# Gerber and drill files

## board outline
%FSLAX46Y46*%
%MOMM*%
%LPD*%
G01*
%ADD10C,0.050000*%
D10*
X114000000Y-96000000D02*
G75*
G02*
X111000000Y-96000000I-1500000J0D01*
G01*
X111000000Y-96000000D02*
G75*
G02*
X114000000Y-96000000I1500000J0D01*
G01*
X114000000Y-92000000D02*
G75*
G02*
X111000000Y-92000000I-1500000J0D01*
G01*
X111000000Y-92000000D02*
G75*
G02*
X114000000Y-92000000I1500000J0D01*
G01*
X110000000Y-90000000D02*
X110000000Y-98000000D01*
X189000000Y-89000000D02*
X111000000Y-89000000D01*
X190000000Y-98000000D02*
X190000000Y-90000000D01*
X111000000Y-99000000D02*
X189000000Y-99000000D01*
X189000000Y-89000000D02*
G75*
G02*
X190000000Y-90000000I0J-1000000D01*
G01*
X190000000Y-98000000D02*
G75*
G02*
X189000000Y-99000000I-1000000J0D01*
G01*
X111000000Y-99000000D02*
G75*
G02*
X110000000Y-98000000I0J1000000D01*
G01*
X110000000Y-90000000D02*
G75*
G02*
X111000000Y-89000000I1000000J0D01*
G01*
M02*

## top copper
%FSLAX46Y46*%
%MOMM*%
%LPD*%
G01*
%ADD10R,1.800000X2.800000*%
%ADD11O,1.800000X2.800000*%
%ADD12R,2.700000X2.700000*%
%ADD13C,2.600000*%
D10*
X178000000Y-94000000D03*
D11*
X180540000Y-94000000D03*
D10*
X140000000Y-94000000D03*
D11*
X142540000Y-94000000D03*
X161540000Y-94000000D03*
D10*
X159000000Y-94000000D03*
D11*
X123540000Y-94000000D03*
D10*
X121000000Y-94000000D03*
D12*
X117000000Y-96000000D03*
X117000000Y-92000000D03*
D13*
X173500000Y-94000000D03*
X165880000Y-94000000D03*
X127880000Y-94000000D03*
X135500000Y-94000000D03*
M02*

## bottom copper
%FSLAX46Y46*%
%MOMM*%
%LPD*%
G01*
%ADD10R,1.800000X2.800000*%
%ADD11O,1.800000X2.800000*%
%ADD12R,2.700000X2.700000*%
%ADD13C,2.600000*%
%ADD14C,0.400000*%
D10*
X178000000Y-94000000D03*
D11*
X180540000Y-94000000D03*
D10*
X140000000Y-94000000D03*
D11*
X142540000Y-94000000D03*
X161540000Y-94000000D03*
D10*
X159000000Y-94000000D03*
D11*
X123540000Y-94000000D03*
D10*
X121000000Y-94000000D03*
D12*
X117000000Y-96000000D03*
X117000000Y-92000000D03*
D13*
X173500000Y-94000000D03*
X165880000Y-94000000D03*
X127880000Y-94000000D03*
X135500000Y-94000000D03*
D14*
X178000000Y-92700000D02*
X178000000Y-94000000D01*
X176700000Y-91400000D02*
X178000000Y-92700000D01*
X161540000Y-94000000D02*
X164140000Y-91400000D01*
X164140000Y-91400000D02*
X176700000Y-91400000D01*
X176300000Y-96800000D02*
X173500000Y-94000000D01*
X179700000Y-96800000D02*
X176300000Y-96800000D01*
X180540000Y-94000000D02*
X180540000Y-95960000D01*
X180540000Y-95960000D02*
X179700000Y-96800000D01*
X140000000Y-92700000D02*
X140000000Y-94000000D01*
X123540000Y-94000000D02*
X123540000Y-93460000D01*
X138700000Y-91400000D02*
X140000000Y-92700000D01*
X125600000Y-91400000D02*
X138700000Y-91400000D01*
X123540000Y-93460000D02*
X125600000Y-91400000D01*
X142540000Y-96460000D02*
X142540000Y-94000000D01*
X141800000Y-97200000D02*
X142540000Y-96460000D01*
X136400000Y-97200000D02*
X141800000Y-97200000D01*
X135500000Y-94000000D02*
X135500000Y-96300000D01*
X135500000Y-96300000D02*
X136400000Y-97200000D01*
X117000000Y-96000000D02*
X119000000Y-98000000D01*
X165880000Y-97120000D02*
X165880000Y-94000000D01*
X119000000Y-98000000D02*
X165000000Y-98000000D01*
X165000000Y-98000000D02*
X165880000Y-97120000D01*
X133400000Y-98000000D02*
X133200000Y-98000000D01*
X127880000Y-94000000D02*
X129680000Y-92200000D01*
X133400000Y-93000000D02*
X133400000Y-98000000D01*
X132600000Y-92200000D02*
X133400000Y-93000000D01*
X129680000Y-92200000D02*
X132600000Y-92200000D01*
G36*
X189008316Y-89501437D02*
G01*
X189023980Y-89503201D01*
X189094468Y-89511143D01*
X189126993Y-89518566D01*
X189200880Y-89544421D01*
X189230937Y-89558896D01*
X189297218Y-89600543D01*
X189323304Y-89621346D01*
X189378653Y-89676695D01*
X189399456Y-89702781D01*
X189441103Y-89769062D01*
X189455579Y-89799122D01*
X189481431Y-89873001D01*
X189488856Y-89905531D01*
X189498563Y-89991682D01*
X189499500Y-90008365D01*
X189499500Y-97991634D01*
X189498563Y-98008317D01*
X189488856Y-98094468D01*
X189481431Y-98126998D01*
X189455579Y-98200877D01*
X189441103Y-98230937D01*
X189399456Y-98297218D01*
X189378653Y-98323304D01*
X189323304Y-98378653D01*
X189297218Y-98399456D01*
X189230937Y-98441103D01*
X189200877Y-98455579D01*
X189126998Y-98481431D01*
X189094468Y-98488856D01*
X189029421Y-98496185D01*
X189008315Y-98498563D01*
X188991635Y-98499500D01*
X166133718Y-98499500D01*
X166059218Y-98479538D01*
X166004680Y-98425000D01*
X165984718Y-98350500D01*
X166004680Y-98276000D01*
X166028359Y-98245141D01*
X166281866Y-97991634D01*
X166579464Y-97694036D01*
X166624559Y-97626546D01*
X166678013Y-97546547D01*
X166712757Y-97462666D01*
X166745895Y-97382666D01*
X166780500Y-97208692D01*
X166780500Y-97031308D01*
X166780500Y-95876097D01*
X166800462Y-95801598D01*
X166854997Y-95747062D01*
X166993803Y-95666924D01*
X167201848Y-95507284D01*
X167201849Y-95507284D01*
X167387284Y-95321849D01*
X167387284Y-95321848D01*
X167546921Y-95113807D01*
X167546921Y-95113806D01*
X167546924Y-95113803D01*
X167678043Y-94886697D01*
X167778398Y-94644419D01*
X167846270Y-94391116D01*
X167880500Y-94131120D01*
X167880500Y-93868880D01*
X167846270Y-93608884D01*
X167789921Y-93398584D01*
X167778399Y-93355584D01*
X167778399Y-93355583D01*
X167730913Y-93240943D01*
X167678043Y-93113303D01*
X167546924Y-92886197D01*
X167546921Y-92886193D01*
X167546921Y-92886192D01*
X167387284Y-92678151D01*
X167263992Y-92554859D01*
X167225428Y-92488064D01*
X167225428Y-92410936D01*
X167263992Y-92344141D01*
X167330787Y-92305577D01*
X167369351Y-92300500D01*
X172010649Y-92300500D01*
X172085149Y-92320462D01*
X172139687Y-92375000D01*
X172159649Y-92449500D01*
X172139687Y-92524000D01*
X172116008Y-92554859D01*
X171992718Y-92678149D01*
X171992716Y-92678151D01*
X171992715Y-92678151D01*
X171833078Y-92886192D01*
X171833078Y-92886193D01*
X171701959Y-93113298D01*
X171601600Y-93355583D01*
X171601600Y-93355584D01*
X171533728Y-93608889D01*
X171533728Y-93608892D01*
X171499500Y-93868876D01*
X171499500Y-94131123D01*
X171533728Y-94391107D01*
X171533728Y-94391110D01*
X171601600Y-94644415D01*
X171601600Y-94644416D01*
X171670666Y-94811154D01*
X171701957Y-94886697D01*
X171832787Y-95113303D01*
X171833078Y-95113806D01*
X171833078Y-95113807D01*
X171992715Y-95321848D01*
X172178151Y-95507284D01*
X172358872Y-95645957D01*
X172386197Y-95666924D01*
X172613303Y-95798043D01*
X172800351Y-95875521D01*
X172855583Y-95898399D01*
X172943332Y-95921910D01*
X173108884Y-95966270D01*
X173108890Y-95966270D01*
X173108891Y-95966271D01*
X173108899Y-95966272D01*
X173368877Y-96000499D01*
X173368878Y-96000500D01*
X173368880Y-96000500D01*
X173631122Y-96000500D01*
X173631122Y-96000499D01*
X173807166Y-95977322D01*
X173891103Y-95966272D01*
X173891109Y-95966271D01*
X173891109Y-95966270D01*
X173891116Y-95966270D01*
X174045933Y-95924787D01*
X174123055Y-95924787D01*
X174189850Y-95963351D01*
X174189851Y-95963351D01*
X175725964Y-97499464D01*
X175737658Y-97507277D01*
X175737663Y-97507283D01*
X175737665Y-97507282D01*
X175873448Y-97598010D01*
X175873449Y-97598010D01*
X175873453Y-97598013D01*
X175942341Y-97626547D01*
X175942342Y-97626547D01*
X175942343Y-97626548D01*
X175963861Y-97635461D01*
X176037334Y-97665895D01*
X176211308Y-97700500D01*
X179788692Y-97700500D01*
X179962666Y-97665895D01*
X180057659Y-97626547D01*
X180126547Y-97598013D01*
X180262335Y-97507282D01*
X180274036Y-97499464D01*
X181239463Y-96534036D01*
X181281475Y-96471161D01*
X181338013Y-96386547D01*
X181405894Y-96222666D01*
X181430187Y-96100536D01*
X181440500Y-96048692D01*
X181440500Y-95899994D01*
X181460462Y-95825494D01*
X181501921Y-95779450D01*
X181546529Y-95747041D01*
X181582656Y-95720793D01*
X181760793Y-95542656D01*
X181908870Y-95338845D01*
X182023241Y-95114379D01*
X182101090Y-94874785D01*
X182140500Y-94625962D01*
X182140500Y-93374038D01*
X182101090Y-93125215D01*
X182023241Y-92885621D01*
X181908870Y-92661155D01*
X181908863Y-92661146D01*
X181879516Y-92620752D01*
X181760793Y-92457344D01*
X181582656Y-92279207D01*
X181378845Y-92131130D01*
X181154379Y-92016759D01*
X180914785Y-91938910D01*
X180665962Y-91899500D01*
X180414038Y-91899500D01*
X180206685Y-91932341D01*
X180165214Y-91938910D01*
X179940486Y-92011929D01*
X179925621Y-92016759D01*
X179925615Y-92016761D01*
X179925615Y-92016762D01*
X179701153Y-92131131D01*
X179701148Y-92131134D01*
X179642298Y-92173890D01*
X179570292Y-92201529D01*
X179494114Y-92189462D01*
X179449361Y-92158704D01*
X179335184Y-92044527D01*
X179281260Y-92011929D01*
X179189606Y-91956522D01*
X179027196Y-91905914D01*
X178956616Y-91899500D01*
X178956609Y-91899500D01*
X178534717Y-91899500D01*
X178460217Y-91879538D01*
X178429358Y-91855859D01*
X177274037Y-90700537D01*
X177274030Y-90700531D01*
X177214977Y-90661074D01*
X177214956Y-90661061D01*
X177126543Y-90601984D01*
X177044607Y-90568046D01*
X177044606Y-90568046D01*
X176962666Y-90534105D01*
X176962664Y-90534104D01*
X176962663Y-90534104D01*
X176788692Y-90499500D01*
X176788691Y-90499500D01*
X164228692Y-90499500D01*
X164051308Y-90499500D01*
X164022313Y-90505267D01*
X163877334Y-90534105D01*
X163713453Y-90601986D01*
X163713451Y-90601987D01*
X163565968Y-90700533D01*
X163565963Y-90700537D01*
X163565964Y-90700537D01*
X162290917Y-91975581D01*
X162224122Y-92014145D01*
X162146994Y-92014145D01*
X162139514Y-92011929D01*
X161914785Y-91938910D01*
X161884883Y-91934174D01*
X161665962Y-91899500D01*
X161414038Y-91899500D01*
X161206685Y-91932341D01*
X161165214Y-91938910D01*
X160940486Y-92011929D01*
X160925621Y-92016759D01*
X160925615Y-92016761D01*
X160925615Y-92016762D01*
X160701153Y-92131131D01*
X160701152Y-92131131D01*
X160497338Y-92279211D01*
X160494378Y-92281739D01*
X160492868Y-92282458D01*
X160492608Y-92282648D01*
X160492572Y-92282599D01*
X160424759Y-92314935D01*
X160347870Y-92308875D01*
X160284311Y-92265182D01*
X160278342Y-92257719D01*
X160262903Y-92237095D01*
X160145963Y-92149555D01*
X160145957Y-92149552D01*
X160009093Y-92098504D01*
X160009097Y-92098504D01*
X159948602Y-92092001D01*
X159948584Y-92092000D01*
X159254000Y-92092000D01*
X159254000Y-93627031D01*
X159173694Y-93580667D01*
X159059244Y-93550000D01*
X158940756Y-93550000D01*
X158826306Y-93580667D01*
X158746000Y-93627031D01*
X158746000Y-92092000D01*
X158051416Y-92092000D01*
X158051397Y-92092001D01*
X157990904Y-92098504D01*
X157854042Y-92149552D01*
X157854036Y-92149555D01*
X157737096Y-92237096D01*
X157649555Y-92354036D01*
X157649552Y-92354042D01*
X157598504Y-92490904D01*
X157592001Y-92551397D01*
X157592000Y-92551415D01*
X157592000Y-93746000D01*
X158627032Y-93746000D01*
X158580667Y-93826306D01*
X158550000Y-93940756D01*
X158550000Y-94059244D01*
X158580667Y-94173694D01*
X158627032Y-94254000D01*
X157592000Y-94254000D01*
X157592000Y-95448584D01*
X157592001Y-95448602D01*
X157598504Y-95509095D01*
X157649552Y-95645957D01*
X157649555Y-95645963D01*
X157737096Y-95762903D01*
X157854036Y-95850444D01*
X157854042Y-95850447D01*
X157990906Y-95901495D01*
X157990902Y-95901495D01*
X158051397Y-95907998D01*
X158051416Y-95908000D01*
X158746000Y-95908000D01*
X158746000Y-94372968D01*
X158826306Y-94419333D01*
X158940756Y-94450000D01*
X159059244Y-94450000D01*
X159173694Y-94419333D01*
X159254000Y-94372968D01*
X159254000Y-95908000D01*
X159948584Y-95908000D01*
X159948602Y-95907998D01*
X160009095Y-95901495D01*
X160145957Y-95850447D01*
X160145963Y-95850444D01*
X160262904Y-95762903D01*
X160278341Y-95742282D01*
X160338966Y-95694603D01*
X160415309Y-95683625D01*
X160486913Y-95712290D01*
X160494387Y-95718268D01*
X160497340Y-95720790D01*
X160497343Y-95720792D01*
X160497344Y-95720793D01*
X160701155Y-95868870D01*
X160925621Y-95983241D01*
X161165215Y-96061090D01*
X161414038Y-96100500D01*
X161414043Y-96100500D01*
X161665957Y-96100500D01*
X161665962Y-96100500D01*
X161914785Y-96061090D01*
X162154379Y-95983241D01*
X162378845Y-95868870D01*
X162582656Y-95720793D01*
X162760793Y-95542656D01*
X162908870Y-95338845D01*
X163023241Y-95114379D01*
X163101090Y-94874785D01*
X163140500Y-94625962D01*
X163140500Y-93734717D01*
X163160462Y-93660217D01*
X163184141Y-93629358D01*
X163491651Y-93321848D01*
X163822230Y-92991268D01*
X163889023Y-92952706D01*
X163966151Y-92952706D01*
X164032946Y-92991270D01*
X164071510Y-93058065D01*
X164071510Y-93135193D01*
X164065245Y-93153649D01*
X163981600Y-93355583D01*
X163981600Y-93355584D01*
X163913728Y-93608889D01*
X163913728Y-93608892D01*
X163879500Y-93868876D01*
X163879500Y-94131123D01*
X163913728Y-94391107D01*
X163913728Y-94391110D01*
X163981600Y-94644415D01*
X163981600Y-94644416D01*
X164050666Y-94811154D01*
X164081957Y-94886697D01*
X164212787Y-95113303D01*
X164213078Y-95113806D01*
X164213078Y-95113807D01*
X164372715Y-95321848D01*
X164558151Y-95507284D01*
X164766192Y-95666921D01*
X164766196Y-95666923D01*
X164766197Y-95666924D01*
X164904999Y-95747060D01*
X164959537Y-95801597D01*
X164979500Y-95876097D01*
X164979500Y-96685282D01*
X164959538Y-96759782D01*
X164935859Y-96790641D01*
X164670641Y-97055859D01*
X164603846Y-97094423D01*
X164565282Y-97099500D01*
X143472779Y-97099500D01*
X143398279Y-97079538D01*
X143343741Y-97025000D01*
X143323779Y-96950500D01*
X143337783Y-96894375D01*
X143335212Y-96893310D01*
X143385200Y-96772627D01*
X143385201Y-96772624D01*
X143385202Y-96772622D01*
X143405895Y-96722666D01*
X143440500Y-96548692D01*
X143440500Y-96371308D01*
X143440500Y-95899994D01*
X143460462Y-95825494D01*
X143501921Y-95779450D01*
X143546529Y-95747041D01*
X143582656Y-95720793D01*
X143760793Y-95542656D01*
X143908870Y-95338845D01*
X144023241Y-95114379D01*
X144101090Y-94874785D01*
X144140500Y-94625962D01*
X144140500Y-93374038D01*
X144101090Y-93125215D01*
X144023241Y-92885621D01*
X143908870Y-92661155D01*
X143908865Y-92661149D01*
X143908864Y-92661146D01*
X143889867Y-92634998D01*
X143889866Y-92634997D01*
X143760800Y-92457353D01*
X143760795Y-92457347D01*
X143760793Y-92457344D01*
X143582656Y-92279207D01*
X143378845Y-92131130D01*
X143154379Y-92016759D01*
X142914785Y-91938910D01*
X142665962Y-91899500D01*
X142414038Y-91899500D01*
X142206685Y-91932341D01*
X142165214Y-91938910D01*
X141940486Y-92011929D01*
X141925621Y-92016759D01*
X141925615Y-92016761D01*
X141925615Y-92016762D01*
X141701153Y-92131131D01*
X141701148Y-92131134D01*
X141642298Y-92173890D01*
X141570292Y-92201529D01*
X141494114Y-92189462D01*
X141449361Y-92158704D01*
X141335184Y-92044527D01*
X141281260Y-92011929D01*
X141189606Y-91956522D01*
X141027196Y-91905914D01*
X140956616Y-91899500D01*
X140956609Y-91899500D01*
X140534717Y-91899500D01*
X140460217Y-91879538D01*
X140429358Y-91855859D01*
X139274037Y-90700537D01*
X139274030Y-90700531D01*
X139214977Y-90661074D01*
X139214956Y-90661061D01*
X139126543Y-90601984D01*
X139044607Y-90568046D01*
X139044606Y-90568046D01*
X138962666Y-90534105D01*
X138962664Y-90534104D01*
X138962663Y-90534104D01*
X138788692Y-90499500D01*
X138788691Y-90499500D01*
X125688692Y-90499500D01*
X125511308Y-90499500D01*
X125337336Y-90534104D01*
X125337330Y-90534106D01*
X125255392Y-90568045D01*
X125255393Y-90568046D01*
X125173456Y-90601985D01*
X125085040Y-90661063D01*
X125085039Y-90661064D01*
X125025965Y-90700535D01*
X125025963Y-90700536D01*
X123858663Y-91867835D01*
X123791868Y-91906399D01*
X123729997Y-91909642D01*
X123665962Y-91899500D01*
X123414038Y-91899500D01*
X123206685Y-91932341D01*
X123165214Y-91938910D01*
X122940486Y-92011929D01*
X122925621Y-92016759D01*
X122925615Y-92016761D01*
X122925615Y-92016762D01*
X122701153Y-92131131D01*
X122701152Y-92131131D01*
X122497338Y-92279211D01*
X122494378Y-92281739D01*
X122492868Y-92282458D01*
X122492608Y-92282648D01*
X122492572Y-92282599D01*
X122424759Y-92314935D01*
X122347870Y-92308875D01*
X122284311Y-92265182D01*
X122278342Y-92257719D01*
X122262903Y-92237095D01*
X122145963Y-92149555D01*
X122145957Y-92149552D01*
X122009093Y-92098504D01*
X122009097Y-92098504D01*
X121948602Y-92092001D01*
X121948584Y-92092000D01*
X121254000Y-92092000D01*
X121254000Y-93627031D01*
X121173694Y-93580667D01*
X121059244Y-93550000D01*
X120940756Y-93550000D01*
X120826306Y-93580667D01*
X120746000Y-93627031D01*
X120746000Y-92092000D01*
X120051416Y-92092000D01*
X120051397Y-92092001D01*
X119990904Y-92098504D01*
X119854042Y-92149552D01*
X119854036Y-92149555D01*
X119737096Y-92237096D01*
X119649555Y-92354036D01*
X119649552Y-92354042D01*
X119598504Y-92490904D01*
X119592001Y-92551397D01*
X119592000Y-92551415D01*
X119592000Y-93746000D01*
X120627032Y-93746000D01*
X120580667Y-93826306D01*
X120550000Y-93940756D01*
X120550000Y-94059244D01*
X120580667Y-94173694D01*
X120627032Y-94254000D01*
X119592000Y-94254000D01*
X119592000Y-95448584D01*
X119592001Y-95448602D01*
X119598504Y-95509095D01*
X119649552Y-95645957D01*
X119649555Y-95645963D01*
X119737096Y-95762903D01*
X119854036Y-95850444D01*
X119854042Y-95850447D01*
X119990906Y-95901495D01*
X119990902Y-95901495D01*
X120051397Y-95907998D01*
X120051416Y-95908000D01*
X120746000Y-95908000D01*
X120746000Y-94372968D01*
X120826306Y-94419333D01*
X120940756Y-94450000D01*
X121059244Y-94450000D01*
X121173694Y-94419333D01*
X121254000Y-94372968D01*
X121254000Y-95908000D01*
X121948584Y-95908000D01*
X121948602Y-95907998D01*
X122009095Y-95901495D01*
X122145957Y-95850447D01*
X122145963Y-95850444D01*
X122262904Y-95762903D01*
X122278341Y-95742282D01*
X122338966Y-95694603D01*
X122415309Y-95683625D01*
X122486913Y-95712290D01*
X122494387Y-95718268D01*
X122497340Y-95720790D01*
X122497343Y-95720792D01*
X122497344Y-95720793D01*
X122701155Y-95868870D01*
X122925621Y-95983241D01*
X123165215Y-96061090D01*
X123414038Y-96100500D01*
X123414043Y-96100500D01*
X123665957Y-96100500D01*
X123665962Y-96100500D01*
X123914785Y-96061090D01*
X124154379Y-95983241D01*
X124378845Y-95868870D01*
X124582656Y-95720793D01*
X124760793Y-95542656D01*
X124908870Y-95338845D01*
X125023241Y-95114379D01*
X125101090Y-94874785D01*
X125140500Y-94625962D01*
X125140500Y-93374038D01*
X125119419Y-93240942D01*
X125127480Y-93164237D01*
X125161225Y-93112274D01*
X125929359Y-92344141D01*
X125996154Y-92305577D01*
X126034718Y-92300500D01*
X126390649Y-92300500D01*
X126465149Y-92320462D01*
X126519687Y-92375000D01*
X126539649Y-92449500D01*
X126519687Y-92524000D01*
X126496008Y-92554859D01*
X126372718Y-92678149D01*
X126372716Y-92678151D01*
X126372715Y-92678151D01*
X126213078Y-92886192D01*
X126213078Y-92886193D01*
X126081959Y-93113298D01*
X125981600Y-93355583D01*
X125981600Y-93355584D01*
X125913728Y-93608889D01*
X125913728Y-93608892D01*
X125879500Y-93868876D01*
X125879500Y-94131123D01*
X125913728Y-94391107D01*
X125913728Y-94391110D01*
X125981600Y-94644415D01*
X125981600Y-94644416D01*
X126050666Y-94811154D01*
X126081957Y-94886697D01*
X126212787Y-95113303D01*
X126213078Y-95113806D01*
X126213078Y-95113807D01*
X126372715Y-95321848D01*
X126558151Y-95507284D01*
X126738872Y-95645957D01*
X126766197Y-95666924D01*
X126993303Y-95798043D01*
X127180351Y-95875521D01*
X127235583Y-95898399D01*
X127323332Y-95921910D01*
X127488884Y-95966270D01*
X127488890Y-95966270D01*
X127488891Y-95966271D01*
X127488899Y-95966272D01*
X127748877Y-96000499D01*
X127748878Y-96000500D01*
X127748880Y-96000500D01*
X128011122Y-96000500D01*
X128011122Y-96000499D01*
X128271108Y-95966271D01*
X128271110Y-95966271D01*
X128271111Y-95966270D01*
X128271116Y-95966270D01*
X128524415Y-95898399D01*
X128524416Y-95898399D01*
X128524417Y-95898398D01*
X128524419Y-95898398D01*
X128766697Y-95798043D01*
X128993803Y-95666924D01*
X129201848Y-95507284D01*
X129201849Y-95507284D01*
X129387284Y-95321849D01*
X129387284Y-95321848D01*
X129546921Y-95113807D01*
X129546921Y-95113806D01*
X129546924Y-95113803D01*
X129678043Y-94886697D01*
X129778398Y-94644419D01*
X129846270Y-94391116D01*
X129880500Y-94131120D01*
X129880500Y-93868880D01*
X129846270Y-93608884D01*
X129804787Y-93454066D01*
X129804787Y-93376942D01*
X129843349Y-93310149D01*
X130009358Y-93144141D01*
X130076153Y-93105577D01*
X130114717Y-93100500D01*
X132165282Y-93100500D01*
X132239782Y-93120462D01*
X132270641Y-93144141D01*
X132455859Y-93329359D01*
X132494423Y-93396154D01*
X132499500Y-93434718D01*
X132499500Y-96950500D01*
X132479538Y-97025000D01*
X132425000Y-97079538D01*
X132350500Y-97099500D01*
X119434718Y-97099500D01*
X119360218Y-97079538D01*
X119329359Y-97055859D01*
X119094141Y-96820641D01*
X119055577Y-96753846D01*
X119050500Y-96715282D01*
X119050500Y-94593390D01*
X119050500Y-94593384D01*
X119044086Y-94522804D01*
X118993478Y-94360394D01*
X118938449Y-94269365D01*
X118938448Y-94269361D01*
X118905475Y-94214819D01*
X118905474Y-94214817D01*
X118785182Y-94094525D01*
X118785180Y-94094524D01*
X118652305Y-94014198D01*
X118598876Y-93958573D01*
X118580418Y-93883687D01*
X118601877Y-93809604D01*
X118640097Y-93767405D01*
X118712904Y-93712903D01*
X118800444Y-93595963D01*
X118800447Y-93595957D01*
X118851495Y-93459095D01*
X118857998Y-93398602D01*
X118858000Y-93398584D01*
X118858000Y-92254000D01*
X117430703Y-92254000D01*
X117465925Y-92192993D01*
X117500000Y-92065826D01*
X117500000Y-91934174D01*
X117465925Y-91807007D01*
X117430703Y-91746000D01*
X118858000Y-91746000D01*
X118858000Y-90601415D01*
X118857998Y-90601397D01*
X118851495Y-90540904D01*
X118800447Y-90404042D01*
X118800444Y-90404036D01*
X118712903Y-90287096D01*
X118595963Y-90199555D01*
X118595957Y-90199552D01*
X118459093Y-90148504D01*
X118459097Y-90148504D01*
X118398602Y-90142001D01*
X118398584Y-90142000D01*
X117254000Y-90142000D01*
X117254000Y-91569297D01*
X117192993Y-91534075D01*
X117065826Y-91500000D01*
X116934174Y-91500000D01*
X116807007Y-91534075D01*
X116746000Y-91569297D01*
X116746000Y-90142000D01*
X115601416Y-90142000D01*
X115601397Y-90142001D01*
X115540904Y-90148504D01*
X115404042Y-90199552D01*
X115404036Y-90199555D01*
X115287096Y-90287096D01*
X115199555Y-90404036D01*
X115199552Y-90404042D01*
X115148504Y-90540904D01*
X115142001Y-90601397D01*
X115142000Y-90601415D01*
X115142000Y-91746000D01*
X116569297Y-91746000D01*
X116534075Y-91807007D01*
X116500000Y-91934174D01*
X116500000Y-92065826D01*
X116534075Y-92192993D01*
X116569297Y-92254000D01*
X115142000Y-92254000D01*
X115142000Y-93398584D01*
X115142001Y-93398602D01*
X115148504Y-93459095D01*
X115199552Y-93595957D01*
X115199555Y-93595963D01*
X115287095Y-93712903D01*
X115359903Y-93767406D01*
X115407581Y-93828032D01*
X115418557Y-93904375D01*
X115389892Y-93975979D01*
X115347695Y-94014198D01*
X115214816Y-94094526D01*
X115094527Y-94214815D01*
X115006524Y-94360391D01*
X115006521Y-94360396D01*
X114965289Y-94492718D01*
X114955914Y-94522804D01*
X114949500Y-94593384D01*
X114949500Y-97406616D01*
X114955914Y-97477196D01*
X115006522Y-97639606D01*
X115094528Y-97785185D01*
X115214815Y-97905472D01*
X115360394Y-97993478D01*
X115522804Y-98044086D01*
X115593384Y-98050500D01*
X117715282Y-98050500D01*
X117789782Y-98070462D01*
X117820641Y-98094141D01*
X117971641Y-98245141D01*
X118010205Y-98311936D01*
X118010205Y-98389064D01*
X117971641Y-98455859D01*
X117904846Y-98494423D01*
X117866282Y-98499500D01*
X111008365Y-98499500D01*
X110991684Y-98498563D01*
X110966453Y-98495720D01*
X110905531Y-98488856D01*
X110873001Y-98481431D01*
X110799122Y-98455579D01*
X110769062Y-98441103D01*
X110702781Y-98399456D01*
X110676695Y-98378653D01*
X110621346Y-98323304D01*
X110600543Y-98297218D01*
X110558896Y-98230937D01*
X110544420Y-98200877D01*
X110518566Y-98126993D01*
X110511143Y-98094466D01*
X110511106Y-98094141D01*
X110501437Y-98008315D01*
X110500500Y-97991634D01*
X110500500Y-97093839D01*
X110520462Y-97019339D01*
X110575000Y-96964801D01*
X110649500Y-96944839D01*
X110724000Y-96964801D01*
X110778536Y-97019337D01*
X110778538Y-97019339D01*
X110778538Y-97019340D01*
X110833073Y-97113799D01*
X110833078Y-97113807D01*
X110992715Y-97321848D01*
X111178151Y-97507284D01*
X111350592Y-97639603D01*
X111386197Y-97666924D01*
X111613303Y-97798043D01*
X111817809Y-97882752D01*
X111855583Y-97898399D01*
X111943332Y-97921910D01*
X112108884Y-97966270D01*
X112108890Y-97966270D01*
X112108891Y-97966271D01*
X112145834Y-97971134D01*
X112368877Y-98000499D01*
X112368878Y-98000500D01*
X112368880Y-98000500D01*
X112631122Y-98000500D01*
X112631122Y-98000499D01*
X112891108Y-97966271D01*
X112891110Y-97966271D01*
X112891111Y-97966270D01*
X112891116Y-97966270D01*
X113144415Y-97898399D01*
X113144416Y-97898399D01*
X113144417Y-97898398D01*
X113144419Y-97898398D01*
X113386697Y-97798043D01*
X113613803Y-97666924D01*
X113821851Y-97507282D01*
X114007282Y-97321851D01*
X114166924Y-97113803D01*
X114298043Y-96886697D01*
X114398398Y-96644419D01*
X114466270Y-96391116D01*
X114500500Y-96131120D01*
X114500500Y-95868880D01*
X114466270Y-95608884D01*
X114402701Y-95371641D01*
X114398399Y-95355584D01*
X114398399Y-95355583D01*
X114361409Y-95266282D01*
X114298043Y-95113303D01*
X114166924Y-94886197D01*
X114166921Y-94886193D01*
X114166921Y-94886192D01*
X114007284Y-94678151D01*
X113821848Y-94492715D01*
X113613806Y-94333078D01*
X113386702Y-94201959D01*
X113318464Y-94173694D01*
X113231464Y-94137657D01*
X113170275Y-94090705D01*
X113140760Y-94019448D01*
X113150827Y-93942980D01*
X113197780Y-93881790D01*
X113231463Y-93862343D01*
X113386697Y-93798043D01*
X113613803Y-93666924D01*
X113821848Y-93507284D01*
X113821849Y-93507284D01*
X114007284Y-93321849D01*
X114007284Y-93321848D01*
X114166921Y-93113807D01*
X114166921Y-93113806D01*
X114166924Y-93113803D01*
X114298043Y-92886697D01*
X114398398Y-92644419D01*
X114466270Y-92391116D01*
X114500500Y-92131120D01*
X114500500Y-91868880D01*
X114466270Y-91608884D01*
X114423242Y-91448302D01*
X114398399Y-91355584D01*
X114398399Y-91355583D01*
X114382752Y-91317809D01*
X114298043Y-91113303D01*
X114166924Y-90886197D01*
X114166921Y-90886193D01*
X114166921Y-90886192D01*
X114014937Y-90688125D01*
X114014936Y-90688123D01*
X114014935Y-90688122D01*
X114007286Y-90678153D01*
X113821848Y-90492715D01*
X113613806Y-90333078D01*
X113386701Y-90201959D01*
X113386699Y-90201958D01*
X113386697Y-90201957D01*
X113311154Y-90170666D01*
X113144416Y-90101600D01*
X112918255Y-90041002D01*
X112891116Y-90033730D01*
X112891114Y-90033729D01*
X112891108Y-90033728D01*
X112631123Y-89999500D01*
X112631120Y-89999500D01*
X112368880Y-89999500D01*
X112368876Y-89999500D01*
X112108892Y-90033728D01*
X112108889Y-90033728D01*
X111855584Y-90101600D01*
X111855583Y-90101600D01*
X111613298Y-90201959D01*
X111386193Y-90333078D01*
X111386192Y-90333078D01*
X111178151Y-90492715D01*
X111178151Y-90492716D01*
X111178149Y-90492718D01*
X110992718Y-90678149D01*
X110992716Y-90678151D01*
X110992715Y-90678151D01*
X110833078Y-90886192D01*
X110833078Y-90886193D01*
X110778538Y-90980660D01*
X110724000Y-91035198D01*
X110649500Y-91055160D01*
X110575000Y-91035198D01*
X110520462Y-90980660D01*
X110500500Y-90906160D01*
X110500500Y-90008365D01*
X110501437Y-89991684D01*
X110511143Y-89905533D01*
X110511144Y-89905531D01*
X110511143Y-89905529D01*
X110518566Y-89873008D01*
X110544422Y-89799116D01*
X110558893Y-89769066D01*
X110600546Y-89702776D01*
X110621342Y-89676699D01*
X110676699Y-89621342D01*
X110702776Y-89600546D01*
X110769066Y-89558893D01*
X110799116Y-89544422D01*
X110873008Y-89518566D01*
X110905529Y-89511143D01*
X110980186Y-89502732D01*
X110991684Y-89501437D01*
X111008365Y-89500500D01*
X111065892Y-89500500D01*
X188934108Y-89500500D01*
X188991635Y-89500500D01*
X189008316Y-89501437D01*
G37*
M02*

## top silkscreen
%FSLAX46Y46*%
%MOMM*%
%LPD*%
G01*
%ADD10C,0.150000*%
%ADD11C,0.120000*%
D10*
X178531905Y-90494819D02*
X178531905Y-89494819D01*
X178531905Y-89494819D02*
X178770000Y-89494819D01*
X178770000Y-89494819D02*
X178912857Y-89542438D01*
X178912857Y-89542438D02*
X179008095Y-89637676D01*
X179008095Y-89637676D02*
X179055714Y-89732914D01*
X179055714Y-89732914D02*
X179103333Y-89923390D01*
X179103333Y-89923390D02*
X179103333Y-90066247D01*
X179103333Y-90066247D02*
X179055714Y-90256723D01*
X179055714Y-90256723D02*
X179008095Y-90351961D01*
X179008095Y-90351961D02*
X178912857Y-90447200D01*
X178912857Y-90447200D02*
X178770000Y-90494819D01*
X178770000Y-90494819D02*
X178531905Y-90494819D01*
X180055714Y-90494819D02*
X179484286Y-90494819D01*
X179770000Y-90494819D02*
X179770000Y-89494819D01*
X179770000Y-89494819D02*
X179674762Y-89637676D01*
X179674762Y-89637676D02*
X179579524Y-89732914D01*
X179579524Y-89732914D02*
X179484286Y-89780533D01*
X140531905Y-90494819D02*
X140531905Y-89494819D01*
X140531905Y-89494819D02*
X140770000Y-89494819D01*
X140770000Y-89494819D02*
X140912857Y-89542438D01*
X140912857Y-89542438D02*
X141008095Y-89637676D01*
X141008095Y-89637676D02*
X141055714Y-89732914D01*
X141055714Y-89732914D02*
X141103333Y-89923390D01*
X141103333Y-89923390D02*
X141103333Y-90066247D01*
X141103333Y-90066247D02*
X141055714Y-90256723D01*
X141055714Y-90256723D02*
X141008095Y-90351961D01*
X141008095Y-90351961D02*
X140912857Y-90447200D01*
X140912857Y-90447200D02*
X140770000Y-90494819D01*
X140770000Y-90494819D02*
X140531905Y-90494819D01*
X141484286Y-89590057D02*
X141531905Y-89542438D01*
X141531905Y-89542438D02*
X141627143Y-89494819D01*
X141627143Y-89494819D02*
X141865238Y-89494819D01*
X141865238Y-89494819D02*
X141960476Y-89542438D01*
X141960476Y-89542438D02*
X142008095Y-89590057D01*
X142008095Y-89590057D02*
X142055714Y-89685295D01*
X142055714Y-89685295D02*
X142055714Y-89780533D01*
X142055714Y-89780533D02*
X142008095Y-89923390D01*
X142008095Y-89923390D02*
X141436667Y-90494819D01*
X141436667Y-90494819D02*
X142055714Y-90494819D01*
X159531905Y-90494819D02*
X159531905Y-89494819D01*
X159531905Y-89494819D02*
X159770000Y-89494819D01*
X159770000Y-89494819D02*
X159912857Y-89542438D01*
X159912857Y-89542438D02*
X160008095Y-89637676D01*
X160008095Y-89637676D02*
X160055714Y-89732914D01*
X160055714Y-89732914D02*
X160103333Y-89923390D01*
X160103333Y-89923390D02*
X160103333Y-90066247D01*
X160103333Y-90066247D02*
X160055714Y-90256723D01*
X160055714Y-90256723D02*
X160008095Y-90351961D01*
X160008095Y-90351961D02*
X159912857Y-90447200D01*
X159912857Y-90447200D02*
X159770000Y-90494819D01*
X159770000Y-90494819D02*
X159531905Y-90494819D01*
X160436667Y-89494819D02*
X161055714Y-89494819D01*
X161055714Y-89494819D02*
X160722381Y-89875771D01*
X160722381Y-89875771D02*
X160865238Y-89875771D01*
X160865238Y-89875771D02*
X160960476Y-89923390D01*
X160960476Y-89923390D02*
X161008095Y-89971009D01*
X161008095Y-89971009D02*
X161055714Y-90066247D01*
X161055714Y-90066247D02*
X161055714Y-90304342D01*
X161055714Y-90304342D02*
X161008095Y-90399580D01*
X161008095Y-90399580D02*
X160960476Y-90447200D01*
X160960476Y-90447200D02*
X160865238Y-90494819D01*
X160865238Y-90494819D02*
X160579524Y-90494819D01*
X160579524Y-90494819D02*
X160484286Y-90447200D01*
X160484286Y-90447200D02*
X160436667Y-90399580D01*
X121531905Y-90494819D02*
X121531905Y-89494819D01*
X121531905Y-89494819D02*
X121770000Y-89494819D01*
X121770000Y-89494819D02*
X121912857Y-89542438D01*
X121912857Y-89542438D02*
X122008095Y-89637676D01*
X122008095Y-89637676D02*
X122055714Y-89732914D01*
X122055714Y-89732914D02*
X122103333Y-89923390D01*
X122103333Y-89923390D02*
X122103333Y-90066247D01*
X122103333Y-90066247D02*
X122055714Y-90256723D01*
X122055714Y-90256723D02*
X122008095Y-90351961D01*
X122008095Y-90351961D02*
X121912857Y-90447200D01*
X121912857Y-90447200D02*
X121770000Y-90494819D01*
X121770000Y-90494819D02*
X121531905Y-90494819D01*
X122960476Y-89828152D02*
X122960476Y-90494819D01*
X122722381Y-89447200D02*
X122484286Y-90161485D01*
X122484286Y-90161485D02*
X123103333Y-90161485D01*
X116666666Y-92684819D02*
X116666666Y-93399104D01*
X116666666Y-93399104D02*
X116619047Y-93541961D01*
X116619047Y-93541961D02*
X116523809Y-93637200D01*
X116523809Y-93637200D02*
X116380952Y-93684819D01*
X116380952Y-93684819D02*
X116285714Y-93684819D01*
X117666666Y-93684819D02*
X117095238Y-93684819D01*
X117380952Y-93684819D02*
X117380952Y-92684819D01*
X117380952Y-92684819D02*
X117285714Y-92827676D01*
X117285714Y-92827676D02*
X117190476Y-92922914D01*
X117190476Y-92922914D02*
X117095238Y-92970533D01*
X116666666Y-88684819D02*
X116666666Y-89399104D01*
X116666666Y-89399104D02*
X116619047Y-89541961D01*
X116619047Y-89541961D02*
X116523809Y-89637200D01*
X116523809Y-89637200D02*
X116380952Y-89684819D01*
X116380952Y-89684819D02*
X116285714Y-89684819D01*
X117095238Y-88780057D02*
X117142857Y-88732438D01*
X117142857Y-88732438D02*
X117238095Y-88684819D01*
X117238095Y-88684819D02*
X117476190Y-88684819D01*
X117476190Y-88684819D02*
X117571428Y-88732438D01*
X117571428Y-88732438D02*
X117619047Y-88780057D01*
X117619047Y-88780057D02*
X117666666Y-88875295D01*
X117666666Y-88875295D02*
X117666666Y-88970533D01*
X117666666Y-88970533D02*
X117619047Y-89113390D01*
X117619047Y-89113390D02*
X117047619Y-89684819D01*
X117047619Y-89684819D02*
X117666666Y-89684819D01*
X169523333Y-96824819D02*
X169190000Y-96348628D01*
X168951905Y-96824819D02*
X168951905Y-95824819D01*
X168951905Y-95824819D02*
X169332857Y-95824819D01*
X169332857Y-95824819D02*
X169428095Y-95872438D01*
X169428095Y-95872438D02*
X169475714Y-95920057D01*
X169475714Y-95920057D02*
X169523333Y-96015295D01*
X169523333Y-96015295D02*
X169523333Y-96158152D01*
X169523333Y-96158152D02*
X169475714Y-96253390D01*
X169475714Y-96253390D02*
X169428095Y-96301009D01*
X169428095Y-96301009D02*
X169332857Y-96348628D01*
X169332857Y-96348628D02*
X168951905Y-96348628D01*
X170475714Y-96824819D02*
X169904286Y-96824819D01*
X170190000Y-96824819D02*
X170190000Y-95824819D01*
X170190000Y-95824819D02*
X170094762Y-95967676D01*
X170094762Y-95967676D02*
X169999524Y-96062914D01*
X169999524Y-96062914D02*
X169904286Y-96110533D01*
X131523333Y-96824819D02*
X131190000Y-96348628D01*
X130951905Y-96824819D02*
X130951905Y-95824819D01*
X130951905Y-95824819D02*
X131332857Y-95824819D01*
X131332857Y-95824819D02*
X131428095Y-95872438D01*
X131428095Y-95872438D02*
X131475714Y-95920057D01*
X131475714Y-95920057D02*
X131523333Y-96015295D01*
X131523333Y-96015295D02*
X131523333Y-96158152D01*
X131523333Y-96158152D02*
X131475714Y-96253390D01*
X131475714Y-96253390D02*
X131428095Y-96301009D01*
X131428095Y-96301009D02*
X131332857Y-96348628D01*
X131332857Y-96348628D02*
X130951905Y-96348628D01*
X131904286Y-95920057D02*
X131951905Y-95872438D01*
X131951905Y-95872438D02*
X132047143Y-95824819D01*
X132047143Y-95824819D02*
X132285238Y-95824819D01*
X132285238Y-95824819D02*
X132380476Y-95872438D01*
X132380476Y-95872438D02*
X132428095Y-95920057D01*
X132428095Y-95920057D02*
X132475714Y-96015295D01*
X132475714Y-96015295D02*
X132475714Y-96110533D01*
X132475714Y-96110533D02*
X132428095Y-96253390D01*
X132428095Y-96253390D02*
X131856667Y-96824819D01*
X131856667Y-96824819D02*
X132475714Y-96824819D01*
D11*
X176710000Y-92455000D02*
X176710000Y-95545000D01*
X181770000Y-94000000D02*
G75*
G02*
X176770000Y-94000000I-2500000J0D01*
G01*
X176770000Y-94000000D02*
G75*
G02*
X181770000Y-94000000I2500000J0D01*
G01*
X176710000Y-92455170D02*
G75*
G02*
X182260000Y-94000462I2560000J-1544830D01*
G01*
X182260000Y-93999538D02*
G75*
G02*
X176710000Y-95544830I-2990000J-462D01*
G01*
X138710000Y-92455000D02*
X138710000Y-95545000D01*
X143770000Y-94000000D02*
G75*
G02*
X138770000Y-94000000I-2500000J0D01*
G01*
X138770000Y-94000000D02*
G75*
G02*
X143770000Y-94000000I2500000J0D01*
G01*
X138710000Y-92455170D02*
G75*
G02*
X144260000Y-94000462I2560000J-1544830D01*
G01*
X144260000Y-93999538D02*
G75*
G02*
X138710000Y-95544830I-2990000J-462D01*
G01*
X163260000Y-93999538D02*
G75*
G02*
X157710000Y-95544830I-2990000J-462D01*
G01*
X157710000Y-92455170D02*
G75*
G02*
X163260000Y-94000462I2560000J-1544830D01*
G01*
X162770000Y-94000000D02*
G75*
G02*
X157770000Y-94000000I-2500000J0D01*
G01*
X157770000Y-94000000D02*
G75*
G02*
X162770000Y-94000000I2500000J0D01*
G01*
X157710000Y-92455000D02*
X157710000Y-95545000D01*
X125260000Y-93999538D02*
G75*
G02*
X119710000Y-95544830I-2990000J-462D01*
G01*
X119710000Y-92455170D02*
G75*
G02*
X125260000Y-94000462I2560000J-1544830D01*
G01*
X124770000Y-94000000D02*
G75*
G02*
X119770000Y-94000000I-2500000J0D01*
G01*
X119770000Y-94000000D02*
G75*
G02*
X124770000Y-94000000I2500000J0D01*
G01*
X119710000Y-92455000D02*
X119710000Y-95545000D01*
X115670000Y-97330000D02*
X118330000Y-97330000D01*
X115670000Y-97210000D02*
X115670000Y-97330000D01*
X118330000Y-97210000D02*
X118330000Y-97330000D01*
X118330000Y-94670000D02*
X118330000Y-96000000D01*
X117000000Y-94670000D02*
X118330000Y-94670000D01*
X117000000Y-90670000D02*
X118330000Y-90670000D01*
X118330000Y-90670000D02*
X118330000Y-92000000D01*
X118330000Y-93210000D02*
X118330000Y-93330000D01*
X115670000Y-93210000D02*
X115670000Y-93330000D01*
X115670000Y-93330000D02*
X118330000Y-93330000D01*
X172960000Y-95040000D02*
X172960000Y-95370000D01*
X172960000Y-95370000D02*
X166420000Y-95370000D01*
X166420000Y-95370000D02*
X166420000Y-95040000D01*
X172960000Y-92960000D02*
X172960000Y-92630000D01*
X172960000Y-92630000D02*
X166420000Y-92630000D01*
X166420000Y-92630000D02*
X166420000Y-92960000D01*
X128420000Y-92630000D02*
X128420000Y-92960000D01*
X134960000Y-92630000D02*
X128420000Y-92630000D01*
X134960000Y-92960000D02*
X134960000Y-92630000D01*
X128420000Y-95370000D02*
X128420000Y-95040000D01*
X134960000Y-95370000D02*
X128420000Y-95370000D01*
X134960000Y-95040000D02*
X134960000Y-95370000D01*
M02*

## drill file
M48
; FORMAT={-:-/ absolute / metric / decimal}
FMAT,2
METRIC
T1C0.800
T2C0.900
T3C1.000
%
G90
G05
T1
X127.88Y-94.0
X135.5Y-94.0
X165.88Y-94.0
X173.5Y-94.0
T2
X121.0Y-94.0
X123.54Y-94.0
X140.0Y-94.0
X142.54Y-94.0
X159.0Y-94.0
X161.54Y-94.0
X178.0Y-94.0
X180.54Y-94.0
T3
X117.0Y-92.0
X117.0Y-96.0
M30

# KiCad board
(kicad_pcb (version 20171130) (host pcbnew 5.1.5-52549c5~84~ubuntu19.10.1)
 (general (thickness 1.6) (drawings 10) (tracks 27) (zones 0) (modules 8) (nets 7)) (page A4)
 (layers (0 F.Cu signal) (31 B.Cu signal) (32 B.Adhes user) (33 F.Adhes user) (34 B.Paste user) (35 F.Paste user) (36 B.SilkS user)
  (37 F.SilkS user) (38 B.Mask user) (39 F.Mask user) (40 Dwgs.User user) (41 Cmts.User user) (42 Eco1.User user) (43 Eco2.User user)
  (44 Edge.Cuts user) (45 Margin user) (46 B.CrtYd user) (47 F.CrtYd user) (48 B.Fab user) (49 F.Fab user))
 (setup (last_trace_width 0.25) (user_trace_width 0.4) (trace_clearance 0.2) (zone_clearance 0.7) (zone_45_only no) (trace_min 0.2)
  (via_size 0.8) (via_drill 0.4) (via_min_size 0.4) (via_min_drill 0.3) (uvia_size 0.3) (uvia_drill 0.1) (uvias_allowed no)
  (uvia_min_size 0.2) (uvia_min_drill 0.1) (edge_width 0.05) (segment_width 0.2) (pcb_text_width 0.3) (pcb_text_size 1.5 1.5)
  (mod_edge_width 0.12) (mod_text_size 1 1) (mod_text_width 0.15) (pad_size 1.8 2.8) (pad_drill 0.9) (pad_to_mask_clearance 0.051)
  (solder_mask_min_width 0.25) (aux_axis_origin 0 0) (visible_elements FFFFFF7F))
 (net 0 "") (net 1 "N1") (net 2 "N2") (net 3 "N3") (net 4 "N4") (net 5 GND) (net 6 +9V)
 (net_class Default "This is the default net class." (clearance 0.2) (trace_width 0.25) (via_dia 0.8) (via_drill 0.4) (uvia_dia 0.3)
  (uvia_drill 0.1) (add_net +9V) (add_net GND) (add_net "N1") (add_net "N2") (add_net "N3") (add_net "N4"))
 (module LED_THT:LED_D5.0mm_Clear (layer F.Cu) (at 178 94)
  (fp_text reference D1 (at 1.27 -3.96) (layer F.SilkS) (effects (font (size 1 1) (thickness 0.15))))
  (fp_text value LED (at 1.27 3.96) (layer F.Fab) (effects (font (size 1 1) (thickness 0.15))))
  (fp_line (start -1.29 -1.545) (end -1.29 1.545) (layer F.SilkS) (width 0.12))
  (fp_circle (center 1.27 0) (end 3.77 0) (layer F.SilkS) (width 0.12))
  (fp_arc (start 1.27 0) (end -1.29 -1.54483) (angle 148.9) (layer F.SilkS) (width 0.12))
  (fp_arc (start 1.27 0) (end -1.29 1.54483) (angle -148.9) (layer F.SilkS) (width 0.12))
  (pad 1 thru_hole rect (at 0 0) (size 1.8 2.8) (drill 0.9) (layers *.Cu *.Mask) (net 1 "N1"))
  (pad 2 thru_hole oval (at 2.54 0) (size 1.8 2.8) (drill 0.9) (layers *.Cu *.Mask) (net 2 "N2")))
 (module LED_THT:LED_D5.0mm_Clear (layer F.Cu) (at 140 94)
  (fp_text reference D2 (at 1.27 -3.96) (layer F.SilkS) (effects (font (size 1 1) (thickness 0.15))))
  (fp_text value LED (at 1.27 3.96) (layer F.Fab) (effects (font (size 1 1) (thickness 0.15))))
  (fp_line (start -1.29 -1.545) (end -1.29 1.545) (layer F.SilkS) (width 0.12))
  (fp_circle (center 1.27 0) (end 3.77 0) (layer F.SilkS) (width 0.12))
  (fp_arc (start 1.27 0) (end -1.29 -1.54483) (angle 148.9) (layer F.SilkS) (width 0.12))
  (fp_arc (start 1.27 0) (end -1.29 1.54483) (angle -148.9) (layer F.SilkS) (width 0.12))
  (pad 1 thru_hole rect (at 0 0) (size 1.8 2.8) (drill 0.9) (layers *.Cu *.Mask) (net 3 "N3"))
  (pad 2 thru_hole oval (at 2.54 0) (size 1.8 2.8) (drill 0.9) (layers *.Cu *.Mask) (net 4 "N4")))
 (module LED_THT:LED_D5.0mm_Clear (layer F.Cu) (at 159 94)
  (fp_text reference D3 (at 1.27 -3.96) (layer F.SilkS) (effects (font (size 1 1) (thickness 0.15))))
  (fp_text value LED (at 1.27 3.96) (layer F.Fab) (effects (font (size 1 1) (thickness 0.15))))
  (fp_arc (start 1.27 0) (end -1.29 1.54483) (angle -148.9) (layer F.SilkS) (width 0.12))
  (fp_arc (start 1.27 0) (end -1.29 -1.54483) (angle 148.9) (layer F.SilkS) (width 0.12))
  (fp_circle (center 1.27 0) (end 3.77 0) (layer F.SilkS) (width 0.12))
  (fp_line (start -1.29 -1.545) (end -1.29 1.545) (layer F.SilkS) (width 0.12))
  (pad 2 thru_hole oval (at 2.54 0) (size 1.8 2.8) (drill 0.9) (layers *.Cu *.Mask) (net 1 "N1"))
  (pad 1 thru_hole rect (at 0 0) (size 1.8 2.8) (drill 0.9) (layers *.Cu *.Mask) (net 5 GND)))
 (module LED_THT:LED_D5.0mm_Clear (layer F.Cu) (at 121 94)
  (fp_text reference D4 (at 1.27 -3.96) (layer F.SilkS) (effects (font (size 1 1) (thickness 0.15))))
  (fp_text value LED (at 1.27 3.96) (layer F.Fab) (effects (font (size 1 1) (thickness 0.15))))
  (fp_arc (start 1.27 0) (end -1.29 1.54483) (angle -148.9) (layer F.SilkS) (width 0.12))
  (fp_arc (start 1.27 0) (end -1.29 -1.54483) (angle 148.9) (layer F.SilkS) (width 0.12))
  (fp_circle (center 1.27 0) (end 3.77 0) (layer F.SilkS) (width 0.12))
  (fp_line (start -1.29 -1.545) (end -1.29 1.545) (layer F.SilkS) (width 0.12))
  (pad 2 thru_hole oval (at 2.54 0) (size 1.8 2.8) (drill 0.9) (layers *.Cu *.Mask) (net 3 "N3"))
  (pad 1 thru_hole rect (at 0 0) (size 1.8 2.8) (drill 0.9) (layers *.Cu *.Mask) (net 5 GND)))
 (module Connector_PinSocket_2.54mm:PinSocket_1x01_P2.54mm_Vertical (layer F.Cu) (at 117 96)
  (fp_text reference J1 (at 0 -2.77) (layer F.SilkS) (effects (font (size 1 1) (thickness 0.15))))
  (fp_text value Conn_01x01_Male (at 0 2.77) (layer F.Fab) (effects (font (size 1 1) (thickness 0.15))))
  (fp_line (start -1.33 1.33) (end 1.33 1.33) (layer F.SilkS) (width 0.12))
  (fp_line (start -1.33 1.21) (end -1.33 1.33) (layer F.SilkS) (width 0.12))
  (fp_line (start 1.33 1.21) (end 1.33 1.33) (layer F.SilkS) (width 0.12))
  (fp_line (start 1.33 -1.33) (end 1.33 0) (layer F.SilkS) (width 0.12))
  (fp_line (start 0 -1.33) (end 1.33 -1.33) (layer F.SilkS) (width 0.12))
  (pad 1 thru_hole rect (at 0 0) (size 2.7 2.7) (drill 1) (layers *.Cu *.Mask) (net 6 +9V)))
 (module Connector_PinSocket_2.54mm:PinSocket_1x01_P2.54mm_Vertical (layer F.Cu) (at 117 92)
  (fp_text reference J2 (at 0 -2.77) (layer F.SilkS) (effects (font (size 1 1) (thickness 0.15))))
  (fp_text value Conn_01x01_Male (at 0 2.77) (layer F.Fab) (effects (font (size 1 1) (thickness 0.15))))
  (fp_line (start 0 -1.33) (end 1.33 -1.33) (layer F.SilkS) (width 0.12))
  (fp_line (start 1.33 -1.33) (end 1.33 0) (layer F.SilkS) (width 0.12))
  (fp_line (start 1.33 1.21) (end 1.33 1.33) (layer F.SilkS) (width 0.12))
  (fp_line (start -1.33 1.21) (end -1.33 1.33) (layer F.SilkS) (width 0.12))
  (fp_line (start -1.33 1.33) (end 1.33 1.33) (layer F.SilkS) (width 0.12))
  (pad 1 thru_hole rect (at 0 0) (size 2.7 2.7) (drill 1) (layers *.Cu *.Mask) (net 5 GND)))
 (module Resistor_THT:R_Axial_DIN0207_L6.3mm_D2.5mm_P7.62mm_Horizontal (layer F.Cu) (at 173.5 94 180)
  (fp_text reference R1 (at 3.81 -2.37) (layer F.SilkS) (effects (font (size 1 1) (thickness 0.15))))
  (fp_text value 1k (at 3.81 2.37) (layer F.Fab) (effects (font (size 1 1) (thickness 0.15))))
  (fp_line (start 0.54 -1.04) (end 0.54 -1.37) (layer F.SilkS) (width 0.12))
  (fp_line (start 0.54 -1.37) (end 7.08 -1.37) (layer F.SilkS) (width 0.12))
  (fp_line (start 7.08 -1.37) (end 7.08 -1.04) (layer F.SilkS) (width 0.12))
  (fp_line (start 0.54 1.04) (end 0.54 1.37) (layer F.SilkS) (width 0.12))
  (fp_line (start 0.54 1.37) (end 7.08 1.37) (layer F.SilkS) (width 0.12))
  (fp_line (start 7.08 1.37) (end 7.08 1.04) (layer F.SilkS) (width 0.12))
  (pad 1 thru_hole circle (at 0 0 180) (size 2.6 2.6) (drill 0.8) (layers *.Cu *.Mask) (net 2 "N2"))
  (pad 2 thru_hole circle (at 7.62 0 180) (size 2.6 2.6) (drill 0.8) (layers *.Cu *.Mask) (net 6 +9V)))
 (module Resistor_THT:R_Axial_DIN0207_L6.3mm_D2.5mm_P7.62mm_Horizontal (layer F.Cu) (at 135.5 94 180)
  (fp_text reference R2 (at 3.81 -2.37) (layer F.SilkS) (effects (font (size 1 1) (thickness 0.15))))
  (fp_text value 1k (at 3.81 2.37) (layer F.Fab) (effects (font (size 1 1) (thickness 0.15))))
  (fp_line (start 7.08 1.37) (end 7.08 1.04) (layer F.SilkS) (width 0.12))
  (fp_line (start 0.54 1.37) (end 7.08 1.37) (layer F.SilkS) (width 0.12))
  (fp_line (start 0.54 1.04) (end 0.54 1.37) (layer F.SilkS) (width 0.12))
  (fp_line (start 7.08 -1.37) (end 7.08 -1.04) (layer F.SilkS) (width 0.12))
  (fp_line (start 0.54 -1.37) (end 7.08 -1.37) (layer F.SilkS) (width 0.12))
  (fp_line (start 0.54 -1.04) (end 0.54 -1.37) (layer F.SilkS) (width 0.12))
  (pad 2 thru_hole circle (at 7.62 0 180) (size 2.6 2.6) (drill 0.8) (layers *.Cu *.Mask) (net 6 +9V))
  (pad 1 thru_hole circle (at 0 0 180) (size 2.6 2.6) (drill 0.8) (layers *.Cu *.Mask) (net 4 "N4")))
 (gr_circle (center 112.5 96) (end 112.5 94.5) (layer Edge.Cuts) (width 0.05))
 (gr_circle (center 112.5 92) (end 112.5 90.5) (layer Edge.Cuts) (width 0.05))
 (gr_line (start 110 90) (end 110 98) (layer Edge.Cuts) (width 0.05))
 (gr_line (start 189 89) (end 111 89) (layer Edge.Cuts) (width 0.05))
 (gr_line (start 190 98) (end 190 90) (layer Edge.Cuts) (width 0.05))
 (gr_line (start 111 99) (end 189 99) (layer Edge.Cuts) (width 0.05))
 (gr_arc (start 189 90) (end 190 90) (angle -90) (layer Edge.Cuts) (width 0.05))
 (gr_arc (start 189 98) (end 189 99) (angle -90) (layer Edge.Cuts) (width 0.05))
 (gr_arc (start 111 98) (end 110 98) (angle -90) (layer Edge.Cuts) (width 0.05))
 (gr_arc (start 111 90) (end 111 89) (angle -90) (layer Edge.Cuts) (width 0.05))
 (segment (start 178 92.7) (end 178 94) (width 0.4) (layer B.Cu) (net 1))
 (segment (start 176.7 91.4) (end 178 92.7) (width 0.4) (layer B.Cu) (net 1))
 (segment (start 161.54 94) (end 164.14 91.4) (width 0.4) (layer B.Cu) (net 1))
 (segment (start 164.14 91.4) (end 176.7 91.4) (width 0.4) (layer B.Cu) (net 1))
 (segment (start 176.3 96.8) (end 173.5 94) (width 0.4) (layer B.Cu) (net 2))
 (segment (start 179.7 96.8) (end 176.3 96.8) (width 0.4) (layer B.Cu) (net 2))
 (segment (start 180.54 94) (end 180.54 95.96) (width 0.4) (layer B.Cu) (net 2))
 (segment (start 180.54 95.96) (end 179.7 96.8) (width 0.4) (layer B.Cu) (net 2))
 (segment (start 140 92.7) (end 140 94) (width 0.4) (layer B.Cu) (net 3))
 (segment (start 123.54 94) (end 123.54 93.46) (width 0.4) (layer B.Cu) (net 3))
 (segment (start 138.7 91.4) (end 140 92.7) (width 0.4) (layer B.Cu) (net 3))
 (segment (start 125.6 91.4) (end 138.7 91.4) (width 0.4) (layer B.Cu) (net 3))
 (segment (start 123.54 93.46) (end 125.6 91.4) (width 0.4) (layer B.Cu) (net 3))
 (segment (start 142.54 96.46) (end 142.54 94) (width 0.4) (layer B.Cu) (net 4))
 (segment (start 141.8 97.2) (end 142.54 96.46) (width 0.4) (layer B.Cu) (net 4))
 (segment (start 136.4 97.2) (end 141.8 97.2) (width 0.4) (layer B.Cu) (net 4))
 (segment (start 135.5 94) (end 135.5 96.3) (width 0.4) (layer B.Cu) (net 4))
 (segment (start 135.5 96.3) (end 136.4 97.2) (width 0.4) (layer B.Cu) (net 4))
 (segment (start 117 96) (end 119 98) (width 0.4) (layer B.Cu) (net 6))
 (segment (start 165.88 97.12) (end 165.88 94) (width 0.4) (layer B.Cu) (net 6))
 (segment (start 119 98) (end 165 98) (width 0.4) (layer B.Cu) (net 6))
 (segment (start 165 98) (end 165.88 97.12) (width 0.4) (layer B.Cu) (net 6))
 (segment (start 133.4 98) (end 133.2 98) (width 0.4) (layer B.Cu) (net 6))
 (segment (start 127.88 94) (end 129.68 92.2) (width 0.4) (layer B.Cu) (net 6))
 (segment (start 133.4 93) (end 133.4 98) (width 0.4) (layer B.Cu) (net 6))
 (segment (start 132.6 92.2) (end 133.4 93) (width 0.4) (layer B.Cu) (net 6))
 (segment (start 129.68 92.2) (end 132.6 92.2) (width 0.4) (layer B.Cu) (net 6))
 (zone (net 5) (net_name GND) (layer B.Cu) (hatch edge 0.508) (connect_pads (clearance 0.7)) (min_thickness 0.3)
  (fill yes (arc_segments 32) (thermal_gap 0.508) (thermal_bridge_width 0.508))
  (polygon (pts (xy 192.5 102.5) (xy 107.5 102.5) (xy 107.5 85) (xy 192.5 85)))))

